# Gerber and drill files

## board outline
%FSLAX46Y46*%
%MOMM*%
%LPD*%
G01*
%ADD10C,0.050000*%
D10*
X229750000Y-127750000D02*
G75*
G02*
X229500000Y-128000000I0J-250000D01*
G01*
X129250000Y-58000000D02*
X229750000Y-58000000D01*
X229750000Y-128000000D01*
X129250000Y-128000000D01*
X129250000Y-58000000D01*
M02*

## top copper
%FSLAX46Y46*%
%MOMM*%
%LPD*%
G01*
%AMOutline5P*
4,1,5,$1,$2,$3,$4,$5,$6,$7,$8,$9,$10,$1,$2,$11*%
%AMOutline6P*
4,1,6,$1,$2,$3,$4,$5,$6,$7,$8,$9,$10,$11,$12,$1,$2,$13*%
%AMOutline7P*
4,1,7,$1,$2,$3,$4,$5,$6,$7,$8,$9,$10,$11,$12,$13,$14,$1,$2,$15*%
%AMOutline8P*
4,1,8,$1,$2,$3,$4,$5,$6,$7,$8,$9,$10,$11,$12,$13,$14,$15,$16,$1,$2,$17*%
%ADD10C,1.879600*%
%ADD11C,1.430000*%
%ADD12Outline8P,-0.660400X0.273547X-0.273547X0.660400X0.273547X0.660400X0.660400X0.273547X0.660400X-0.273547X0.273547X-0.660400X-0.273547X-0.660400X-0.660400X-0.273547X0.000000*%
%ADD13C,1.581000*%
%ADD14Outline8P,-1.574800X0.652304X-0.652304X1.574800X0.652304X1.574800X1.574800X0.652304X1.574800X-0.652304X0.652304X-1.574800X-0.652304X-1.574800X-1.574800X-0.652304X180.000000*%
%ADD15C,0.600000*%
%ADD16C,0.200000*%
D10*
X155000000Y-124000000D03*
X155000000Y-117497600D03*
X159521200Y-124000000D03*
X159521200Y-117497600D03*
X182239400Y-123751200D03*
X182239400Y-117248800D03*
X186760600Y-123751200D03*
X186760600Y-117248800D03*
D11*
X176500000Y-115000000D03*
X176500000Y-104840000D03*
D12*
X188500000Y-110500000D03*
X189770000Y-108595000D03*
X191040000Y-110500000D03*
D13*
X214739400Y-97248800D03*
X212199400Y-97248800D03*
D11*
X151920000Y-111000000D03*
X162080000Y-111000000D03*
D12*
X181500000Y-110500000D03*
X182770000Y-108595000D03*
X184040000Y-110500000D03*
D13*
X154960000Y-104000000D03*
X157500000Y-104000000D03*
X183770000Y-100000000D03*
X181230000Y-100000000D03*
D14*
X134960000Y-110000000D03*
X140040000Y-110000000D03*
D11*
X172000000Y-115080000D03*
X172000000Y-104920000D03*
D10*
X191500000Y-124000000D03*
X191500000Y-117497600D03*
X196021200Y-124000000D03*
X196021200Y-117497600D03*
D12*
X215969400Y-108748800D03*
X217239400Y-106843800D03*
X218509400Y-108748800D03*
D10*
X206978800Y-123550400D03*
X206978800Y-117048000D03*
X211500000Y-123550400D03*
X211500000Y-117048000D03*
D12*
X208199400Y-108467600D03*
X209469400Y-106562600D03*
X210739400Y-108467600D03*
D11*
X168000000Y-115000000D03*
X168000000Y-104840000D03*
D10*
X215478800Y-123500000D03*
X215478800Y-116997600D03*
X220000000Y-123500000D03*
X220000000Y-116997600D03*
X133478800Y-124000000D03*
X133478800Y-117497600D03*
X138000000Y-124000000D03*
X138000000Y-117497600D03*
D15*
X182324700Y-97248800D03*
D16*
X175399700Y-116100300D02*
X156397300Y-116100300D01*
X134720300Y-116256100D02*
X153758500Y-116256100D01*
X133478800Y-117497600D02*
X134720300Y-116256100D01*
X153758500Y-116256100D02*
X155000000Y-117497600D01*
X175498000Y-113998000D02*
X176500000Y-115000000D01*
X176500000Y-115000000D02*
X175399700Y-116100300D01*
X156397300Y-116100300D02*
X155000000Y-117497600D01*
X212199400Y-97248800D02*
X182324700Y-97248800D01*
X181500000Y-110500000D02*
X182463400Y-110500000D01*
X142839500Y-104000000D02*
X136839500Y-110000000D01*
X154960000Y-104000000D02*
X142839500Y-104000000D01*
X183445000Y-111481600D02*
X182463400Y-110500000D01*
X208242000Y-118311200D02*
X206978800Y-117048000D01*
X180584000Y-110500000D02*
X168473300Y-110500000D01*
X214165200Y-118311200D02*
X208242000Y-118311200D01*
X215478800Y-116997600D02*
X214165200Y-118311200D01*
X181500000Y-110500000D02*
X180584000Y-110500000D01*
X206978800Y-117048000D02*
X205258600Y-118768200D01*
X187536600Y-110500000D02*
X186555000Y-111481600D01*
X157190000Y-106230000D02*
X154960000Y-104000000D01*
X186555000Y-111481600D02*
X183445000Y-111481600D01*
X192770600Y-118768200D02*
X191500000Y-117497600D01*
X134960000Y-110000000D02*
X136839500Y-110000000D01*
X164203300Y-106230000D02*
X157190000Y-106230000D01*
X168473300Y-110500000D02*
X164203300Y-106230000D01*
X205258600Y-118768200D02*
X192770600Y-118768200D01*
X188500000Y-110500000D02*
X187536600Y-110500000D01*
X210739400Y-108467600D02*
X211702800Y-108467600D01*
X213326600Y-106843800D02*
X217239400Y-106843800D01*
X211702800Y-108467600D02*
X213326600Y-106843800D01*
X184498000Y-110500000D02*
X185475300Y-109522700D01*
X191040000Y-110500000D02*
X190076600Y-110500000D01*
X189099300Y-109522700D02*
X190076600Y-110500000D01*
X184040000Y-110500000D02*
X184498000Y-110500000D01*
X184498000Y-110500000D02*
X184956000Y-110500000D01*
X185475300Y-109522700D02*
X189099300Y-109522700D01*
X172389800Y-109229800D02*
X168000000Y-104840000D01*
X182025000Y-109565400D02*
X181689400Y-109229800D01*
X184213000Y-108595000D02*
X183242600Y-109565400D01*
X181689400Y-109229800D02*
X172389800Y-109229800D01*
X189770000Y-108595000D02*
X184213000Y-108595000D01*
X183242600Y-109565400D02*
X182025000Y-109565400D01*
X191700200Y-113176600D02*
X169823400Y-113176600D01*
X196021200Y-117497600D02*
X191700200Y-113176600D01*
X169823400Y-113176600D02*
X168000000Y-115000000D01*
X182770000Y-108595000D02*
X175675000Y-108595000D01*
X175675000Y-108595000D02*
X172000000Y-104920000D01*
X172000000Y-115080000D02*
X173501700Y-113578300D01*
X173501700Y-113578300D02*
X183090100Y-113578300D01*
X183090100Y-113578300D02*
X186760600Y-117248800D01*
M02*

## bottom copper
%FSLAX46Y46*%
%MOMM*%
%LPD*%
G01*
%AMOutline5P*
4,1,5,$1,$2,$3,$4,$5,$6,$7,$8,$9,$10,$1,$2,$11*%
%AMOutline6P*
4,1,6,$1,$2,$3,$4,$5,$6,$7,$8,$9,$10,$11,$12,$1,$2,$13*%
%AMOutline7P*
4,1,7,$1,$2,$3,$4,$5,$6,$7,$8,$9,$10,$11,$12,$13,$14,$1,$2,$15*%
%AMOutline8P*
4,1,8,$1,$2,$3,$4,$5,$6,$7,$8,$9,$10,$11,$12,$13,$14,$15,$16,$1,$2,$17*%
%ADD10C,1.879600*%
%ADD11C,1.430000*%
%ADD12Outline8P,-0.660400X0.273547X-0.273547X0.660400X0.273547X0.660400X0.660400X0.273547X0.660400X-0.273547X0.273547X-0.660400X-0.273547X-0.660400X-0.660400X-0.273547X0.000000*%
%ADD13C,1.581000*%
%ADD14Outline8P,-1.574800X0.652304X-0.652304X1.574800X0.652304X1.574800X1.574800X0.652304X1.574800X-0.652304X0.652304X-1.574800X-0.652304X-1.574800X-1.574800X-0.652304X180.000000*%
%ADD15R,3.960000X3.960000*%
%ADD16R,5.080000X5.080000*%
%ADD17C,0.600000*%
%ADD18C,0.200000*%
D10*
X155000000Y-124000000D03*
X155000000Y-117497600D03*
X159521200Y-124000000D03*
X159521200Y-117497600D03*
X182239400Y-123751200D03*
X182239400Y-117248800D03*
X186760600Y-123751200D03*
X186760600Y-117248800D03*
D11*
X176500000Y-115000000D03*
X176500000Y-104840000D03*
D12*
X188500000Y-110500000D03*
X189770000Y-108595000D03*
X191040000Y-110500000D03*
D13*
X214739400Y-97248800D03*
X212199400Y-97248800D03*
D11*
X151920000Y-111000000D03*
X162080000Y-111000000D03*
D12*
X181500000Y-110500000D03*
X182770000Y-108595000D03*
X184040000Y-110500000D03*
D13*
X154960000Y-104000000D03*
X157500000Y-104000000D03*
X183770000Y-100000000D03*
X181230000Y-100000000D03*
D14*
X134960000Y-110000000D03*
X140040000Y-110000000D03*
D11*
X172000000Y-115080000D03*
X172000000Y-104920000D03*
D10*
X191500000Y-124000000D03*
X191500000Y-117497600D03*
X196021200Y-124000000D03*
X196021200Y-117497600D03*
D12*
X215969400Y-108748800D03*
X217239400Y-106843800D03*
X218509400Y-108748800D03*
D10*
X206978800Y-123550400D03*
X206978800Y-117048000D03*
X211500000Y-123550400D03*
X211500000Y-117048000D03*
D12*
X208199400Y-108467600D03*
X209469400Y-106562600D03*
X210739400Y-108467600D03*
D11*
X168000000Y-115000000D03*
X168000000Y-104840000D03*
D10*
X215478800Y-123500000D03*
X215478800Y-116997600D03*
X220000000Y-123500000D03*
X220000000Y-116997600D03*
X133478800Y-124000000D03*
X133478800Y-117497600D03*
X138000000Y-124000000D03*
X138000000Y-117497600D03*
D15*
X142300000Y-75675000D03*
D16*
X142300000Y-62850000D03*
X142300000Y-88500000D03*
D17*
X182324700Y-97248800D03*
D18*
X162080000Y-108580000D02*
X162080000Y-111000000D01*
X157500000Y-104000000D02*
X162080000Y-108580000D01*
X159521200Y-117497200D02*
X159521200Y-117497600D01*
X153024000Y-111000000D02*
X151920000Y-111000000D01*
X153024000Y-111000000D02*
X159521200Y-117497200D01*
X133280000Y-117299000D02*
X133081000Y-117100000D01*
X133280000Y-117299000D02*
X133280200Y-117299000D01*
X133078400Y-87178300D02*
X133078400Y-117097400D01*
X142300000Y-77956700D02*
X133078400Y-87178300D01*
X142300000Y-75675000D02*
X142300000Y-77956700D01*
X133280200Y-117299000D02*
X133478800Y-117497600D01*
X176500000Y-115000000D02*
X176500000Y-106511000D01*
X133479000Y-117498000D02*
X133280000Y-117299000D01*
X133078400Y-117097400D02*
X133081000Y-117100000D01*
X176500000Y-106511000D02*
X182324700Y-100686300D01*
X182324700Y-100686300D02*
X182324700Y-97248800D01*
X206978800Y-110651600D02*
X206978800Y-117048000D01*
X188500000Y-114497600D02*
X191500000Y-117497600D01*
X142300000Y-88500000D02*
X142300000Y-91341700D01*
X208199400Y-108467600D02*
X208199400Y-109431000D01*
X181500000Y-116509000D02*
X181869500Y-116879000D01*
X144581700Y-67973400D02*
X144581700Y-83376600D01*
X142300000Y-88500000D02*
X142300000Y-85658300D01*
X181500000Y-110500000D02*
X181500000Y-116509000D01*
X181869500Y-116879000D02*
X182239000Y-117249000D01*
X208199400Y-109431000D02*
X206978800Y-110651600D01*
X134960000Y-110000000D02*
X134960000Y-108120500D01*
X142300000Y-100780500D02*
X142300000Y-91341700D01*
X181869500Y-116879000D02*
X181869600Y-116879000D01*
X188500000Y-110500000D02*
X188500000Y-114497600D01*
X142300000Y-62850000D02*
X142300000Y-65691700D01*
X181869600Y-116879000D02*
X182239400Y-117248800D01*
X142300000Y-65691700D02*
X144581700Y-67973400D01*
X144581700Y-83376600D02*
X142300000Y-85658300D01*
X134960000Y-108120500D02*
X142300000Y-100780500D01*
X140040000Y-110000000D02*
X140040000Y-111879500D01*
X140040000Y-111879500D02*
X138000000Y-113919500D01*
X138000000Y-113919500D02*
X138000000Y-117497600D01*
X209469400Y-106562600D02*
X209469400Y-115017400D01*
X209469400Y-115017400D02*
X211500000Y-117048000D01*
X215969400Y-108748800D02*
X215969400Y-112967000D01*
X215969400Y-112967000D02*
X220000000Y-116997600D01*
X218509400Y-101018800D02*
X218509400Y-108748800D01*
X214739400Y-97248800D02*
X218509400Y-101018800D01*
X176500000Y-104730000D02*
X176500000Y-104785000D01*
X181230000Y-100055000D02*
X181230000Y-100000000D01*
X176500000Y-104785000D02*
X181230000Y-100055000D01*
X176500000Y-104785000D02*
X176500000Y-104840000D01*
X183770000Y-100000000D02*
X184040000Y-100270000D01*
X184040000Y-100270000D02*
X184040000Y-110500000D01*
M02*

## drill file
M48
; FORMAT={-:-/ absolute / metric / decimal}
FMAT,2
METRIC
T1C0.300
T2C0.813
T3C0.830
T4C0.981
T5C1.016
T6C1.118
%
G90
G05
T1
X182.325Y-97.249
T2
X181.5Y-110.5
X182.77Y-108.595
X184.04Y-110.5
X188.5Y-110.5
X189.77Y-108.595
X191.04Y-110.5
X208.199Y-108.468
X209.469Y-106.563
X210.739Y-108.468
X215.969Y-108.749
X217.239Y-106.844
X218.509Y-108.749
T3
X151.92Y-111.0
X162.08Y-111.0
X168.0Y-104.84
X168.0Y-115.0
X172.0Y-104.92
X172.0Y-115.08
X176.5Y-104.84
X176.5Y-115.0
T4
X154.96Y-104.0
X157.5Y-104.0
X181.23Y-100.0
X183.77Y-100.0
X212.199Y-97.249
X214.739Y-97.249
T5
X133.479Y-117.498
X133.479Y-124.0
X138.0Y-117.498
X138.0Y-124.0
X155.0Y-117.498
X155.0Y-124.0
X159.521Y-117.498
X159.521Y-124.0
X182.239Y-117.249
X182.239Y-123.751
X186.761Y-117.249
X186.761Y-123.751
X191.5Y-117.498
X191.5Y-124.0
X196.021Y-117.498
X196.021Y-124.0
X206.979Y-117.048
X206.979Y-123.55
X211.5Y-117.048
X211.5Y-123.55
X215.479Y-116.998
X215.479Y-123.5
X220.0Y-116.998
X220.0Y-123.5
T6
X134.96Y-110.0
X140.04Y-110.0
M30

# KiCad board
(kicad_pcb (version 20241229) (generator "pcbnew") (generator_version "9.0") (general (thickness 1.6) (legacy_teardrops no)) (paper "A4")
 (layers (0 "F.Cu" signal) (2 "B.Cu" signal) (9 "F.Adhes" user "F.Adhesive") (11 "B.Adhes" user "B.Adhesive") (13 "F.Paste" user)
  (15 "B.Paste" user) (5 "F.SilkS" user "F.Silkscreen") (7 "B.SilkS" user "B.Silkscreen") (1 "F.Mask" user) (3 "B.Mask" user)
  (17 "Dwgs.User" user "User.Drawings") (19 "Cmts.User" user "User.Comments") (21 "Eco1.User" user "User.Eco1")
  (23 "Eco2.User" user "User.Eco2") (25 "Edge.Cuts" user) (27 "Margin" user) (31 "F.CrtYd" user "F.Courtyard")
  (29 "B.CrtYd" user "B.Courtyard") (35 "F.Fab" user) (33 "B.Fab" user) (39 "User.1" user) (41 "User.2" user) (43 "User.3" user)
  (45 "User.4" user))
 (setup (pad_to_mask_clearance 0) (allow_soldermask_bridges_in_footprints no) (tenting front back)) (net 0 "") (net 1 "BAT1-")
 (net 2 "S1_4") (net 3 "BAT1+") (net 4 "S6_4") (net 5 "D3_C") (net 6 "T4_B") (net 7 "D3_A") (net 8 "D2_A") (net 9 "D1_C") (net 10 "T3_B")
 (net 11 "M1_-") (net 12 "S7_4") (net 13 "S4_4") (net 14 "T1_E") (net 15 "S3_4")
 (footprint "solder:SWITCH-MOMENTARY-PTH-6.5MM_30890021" (layer "F.Cu") (at 157.2606 120.7488 90)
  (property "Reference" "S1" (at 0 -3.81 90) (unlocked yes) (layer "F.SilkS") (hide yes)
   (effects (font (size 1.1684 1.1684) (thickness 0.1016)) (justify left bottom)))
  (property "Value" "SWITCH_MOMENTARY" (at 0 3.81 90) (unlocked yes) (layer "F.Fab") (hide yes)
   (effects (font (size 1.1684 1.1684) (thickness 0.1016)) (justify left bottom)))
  (pad "1" thru_hole circle (at -3.2512 -2.2606 90) (size 1.8796 1.8796) (drill 1.016) (layers "*.Cu" "*.Mask") (remove_unused_layers no)
   (solder_mask_margin 0.1016) (thermal_bridge_angle 0))
  (pad "2" thru_hole circle (at 3.2512 -2.2606 90) (size 1.8796 1.8796) (drill 1.016) (layers "*.Cu" "*.Mask") (remove_unused_layers no)
   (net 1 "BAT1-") (solder_mask_margin 0.1016) (thermal_bridge_angle 0))
  (pad "3" thru_hole circle (at -3.2512 2.2606 90) (size 1.8796 1.8796) (drill 1.016) (layers "*.Cu" "*.Mask") (remove_unused_layers no)
   (solder_mask_margin 0.1016) (thermal_bridge_angle 0))
  (pad "4" thru_hole circle (at 3.2512 2.2606 90) (size 1.8796 1.8796) (drill 1.016) (layers "*.Cu" "*.Mask") (remove_unused_layers no)
   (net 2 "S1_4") (solder_mask_margin 0.1016) (thermal_bridge_angle 0)))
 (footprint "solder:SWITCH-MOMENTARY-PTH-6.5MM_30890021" (layer "F.Cu") (at 184.5 120.5 90)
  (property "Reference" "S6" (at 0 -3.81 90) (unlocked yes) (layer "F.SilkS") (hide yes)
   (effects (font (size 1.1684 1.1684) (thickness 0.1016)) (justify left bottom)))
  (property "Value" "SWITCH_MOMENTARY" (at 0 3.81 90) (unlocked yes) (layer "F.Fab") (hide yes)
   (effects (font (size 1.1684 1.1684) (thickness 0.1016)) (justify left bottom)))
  (pad "1" thru_hole circle (at -3.2512 -2.2606 90) (size 1.8796 1.8796) (drill 1.016) (layers "*.Cu" "*.Mask") (remove_unused_layers no)
   (solder_mask_margin 0.1016) (thermal_bridge_angle 0))
  (pad "2" thru_hole circle (at 3.2512 -2.2606 90) (size 1.8796 1.8796) (drill 1.016) (layers "*.Cu" "*.Mask") (remove_unused_layers no)
   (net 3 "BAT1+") (solder_mask_margin 0.1016) (thermal_bridge_angle 0))
  (pad "3" thru_hole circle (at -3.2512 2.2606 90) (size 1.8796 1.8796) (drill 1.016) (layers "*.Cu" "*.Mask") (remove_unused_layers no)
   (solder_mask_margin 0.1016) (thermal_bridge_angle 0))
  (pad "4" thru_hole circle (at 3.2512 2.2606 90) (size 1.8796 1.8796) (drill 1.016) (layers "*.Cu" "*.Mask") (remove_unused_layers no)
   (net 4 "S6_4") (solder_mask_margin 0.1016) (thermal_bridge_angle 0)))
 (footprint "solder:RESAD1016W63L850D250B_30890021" (layer "F.Cu") (at 176.5 109.92 90)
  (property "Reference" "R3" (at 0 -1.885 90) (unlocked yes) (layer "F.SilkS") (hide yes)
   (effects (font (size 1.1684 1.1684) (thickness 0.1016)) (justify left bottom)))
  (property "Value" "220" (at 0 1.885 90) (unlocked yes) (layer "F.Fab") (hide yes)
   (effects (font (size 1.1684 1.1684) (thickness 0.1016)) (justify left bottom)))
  (pad "1" thru_hole circle (at -5.08 0 90) (size 1.43 1.43) (drill 0.83) (layers "*.Cu" "*.Mask") (remove_unused_layers no) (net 1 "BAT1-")
   (solder_mask_margin 0.1016) (thermal_bridge_angle 0))
  (pad "2" thru_hole circle (at 5.08 0 90) (size 1.43 1.43) (drill 0.83) (layers "*.Cu" "*.Mask") (remove_unused_layers no) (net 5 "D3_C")
   (solder_mask_margin 0.1016) (thermal_bridge_angle 0)))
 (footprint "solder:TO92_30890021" (layer "F.Cu") (at 189.77 110.5)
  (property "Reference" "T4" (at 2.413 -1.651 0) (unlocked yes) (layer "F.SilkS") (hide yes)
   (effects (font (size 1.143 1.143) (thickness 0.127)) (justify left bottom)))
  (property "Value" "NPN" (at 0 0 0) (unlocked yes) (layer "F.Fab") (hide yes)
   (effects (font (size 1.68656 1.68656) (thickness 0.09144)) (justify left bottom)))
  (pad "1" thru_hole roundrect (at -1.27 0) (size 1.3208 1.3208) (drill 0.8128) (layers "*.Cu" "*.Mask") (remove_unused_layers no)
   (roundrect_rratio 0.25) (chamfer_ratio 0.2928932188) (chamfer top_left top_right bottom_left bottom_right) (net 3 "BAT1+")
   (solder_mask_margin 0.1016) (thermal_bridge_angle 0))
  (pad "2" thru_hole roundrect (at 0 -1.905) (size 1.3208 1.3208) (drill 0.8128) (layers "*.Cu" "*.Mask") (remove_unused_layers no)
   (roundrect_rratio 0.25) (chamfer_ratio 0.2928932188) (chamfer top_left top_right bottom_left bottom_right) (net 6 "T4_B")
   (solder_mask_margin 0.1016) (thermal_bridge_angle 0))
  (pad "3" thru_hole roundrect (at 1.27 0) (size 1.3208 1.3208) (drill 0.8128) (layers "*.Cu" "*.Mask") (remove_unused_layers no)
   (roundrect_rratio 0.25) (chamfer_ratio 0.2928932188) (chamfer top_left top_right bottom_left bottom_right) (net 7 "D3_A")
   (solder_mask_margin 0.1016) (thermal_bridge_angle 0)))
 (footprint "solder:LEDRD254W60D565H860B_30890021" (layer "F.Cu") (at 213.4694 97.2488 180)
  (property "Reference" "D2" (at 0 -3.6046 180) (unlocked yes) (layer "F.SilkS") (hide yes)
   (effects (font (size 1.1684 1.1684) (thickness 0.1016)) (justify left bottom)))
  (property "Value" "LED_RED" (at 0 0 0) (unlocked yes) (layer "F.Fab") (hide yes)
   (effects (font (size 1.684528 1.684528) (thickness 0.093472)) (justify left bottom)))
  (pad "1" thru_hole circle (at -1.27 0 180) (size 1.581 1.581) (drill 0.981) (layers "*.Cu" "*.Mask") (remove_unused_layers no)
   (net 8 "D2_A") (solder_mask_margin 0.1016) (thermal_bridge_angle 0))
  (pad "2" thru_hole circle (at 1.27 0 180) (size 1.581 1.581) (drill 0.981) (layers "*.Cu" "*.Mask") (remove_unused_layers no)
   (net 1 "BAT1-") (solder_mask_margin 0.1016) (thermal_bridge_angle 0)))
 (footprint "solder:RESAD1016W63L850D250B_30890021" (layer "F.Cu") (at 157 111)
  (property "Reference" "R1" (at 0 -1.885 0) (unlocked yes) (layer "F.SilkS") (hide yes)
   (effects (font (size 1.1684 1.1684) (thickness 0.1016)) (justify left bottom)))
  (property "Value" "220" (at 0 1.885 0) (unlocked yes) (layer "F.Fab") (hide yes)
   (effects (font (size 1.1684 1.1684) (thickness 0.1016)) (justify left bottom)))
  (pad "1" thru_hole circle (at -5.08 0) (size 1.43 1.43) (drill 0.83) (layers "*.Cu" "*.Mask") (remove_unused_layers no) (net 2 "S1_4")
   (solder_mask_margin 0.1016) (thermal_bridge_angle 0))
  (pad "2" thru_hole circle (at 5.08 0) (size 1.43 1.43) (drill 0.83) (layers "*.Cu" "*.Mask") (remove_unused_layers no) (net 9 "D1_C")
   (solder_mask_margin 0.1016) (thermal_bridge_angle 0)))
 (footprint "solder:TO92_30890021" (layer "F.Cu") (at 182.77 110.5)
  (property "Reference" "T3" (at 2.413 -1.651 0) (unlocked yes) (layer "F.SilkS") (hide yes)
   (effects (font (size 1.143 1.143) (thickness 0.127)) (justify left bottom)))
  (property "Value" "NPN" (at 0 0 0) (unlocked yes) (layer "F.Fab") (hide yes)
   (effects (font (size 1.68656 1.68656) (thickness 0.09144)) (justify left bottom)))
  (pad "1" thru_hole roundrect (at -1.27 0) (size 1.3208 1.3208) (drill 0.8128) (layers "*.Cu" "*.Mask") (remove_unused_layers no)
   (roundrect_rratio 0.25) (chamfer_ratio 0.2928932188) (chamfer top_left top_right bottom_left bottom_right) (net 3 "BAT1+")
   (solder_mask_margin 0.1016) (thermal_bridge_angle 0))
  (pad "2" thru_hole roundrect (at 0 -1.905) (size 1.3208 1.3208) (drill 0.8128) (layers "*.Cu" "*.Mask") (remove_unused_layers no)
   (roundrect_rratio 0.25) (chamfer_ratio 0.2928932188) (chamfer top_left top_right bottom_left bottom_right) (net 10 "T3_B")
   (solder_mask_margin 0.1016) (thermal_bridge_angle 0))
  (pad "3" thru_hole roundrect (at 1.27 0) (size 1.3208 1.3208) (drill 0.8128) (layers "*.Cu" "*.Mask") (remove_unused_layers no)
   (roundrect_rratio 0.25) (chamfer_ratio 0.2928932188) (chamfer top_left top_right bottom_left bottom_right) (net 7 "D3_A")
   (solder_mask_margin 0.1016) (thermal_bridge_angle 0)))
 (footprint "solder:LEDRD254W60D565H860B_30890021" (layer "F.Cu") (at 156.23 104)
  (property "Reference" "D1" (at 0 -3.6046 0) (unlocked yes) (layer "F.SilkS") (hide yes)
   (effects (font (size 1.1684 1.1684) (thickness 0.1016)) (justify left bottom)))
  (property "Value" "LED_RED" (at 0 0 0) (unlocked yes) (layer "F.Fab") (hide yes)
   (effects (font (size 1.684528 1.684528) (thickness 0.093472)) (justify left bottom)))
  (pad "1" thru_hole circle (at -1.27 0) (size 1.581 1.581) (drill 0.981) (layers "*.Cu" "*.Mask") (remove_unused_layers no) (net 3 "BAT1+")
   (solder_mask_margin 0.1016) (thermal_bridge_angle 0))
  (pad "2" thru_hole circle (at 1.27 0) (size 1.581 1.581) (drill 0.981) (layers "*.Cu" "*.Mask") (remove_unused_layers no) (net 9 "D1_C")
   (solder_mask_margin 0.1016) (thermal_bridge_angle 0)))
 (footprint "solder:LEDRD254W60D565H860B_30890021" (layer "F.Cu") (at 182.5 100 180)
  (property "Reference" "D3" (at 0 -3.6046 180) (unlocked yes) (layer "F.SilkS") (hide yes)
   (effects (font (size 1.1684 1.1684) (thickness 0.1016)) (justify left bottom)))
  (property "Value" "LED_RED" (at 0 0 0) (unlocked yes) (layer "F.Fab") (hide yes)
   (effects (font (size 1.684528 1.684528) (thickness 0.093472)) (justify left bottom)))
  (pad "1" thru_hole circle (at -1.27 0 180) (size 1.581 1.581) (drill 0.981) (layers "*.Cu" "*.Mask") (remove_unused_layers no)
   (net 7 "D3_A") (solder_mask_margin 0.1016) (thermal_bridge_angle 0))
  (pad "2" thru_hole circle (at 1.27 0 180) (size 1.581 1.581) (drill 0.981) (layers "*.Cu" "*.Mask") (remove_unused_layers no)
   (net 5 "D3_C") (solder_mask_margin 0.1016) (thermal_bridge_angle 0)))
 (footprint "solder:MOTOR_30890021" (layer "F.Cu") (at 137.5 110 180)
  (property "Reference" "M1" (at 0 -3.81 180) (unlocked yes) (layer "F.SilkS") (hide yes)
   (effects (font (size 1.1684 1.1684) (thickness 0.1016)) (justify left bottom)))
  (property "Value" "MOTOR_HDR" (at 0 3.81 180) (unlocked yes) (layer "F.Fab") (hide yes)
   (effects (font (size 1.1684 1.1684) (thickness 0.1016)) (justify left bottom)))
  (pad "+" thru_hole roundrect (at 2.54 0 180) (size 3.1496 3.1496) (drill 1.1176) (layers "*.Cu" "*.Mask") (remove_unused_layers no)
   (roundrect_rratio 0.25) (chamfer_ratio 0.2928932188) (chamfer top_left top_right bottom_left bottom_right) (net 3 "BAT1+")
   (solder_mask_margin 0.1016) (thermal_bridge_angle 0))
  (pad "-" thru_hole roundrect (at -2.54 0 180) (size 3.1496 3.1496) (drill 1.1176) (layers "*.Cu" "*.Mask") (remove_unused_layers no)
   (roundrect_rratio 0.25) (chamfer_ratio 0.2928932188) (chamfer top_left top_right bottom_left bottom_right) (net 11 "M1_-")
   (solder_mask_margin 0.1016) (thermal_bridge_angle 0)))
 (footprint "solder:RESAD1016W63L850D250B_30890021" (layer "F.Cu") (at 172 110 90)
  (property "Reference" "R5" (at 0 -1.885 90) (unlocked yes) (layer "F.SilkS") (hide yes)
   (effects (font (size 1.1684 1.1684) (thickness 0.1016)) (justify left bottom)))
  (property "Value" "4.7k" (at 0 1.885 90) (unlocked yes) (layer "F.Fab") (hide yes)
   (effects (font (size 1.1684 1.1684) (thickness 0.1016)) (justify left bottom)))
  (pad "1" thru_hole circle (at -5.08 0 90) (size 1.43 1.43) (drill 0.83) (layers "*.Cu" "*.Mask") (remove_unused_layers no) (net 4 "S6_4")
   (solder_mask_margin 0.1016) (thermal_bridge_angle 0))
  (pad "2" thru_hole circle (at 5.08 0 90) (size 1.43 1.43) (drill 0.83) (layers "*.Cu" "*.Mask") (remove_unused_layers no) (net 10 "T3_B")
   (solder_mask_margin 0.1016) (thermal_bridge_angle 0)))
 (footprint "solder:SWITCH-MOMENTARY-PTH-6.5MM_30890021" (layer "F.Cu") (at 193.7606 120.7488 90)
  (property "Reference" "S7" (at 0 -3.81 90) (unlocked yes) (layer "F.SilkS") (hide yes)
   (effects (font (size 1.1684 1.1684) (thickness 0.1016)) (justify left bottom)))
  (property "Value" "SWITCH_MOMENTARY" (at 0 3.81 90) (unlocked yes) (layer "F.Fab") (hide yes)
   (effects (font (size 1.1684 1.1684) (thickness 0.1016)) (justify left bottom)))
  (pad "1" thru_hole circle (at -3.2512 -2.2606 90) (size 1.8796 1.8796) (drill 1.016) (layers "*.Cu" "*.Mask") (remove_unused_layers no)
   (solder_mask_margin 0.1016) (thermal_bridge_angle 0))
  (pad "2" thru_hole circle (at 3.2512 -2.2606 90) (size 1.8796 1.8796) (drill 1.016) (layers "*.Cu" "*.Mask") (remove_unused_layers no)
   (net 3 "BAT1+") (solder_mask_margin 0.1016) (thermal_bridge_angle 0))
  (pad "3" thru_hole circle (at -3.2512 2.2606 90) (size 1.8796 1.8796) (drill 1.016) (layers "*.Cu" "*.Mask") (remove_unused_layers no)
   (solder_mask_margin 0.1016) (thermal_bridge_angle 0))
  (pad "4" thru_hole circle (at 3.2512 2.2606 90) (size 1.8796 1.8796) (drill 1.016) (layers "*.Cu" "*.Mask") (remove_unused_layers no)
   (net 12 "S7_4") (solder_mask_margin 0.1016) (thermal_bridge_angle 0)))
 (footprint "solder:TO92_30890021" (layer "F.Cu") (at 217.2394 108.7488)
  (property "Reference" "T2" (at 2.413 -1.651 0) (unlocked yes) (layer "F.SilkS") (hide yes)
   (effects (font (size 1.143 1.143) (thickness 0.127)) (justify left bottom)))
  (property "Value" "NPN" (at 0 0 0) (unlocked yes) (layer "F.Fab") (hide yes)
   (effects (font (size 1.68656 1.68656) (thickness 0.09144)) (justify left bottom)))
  (pad "1" thru_hole roundrect (at -1.27 0) (size 1.3208 1.3208) (drill 0.8128) (layers "*.Cu" "*.Mask") (remove_unused_layers no)
   (roundrect_rratio 0.25) (chamfer_ratio 0.2928932188) (chamfer top_left top_right bottom_left bottom_right) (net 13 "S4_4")
   (solder_mask_margin 0.1016) (thermal_bridge_angle 0))
  (pad "2" thru_hole roundrect (at 0 -1.905) (size 1.3208 1.3208) (drill 0.8128) (layers "*.Cu" "*.Mask") (remove_unused_layers no)
   (roundrect_rratio 0.25) (chamfer_ratio 0.2928932188) (chamfer top_left top_right bottom_left bottom_right) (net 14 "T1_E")
   (solder_mask_margin 0.1016) (thermal_bridge_angle 0))
  (pad "3" thru_hole roundrect (at 1.27 0) (size 1.3208 1.3208) (drill 0.8128) (layers "*.Cu" "*.Mask") (remove_unused_layers no)
   (roundrect_rratio 0.25) (chamfer_ratio 0.2928932188) (chamfer top_left top_right bottom_left bottom_right) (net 8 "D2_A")
   (solder_mask_margin 0.1016) (thermal_bridge_angle 0)))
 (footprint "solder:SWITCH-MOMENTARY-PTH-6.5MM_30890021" (layer "F.Cu") (at 209.2394 120.2992 90)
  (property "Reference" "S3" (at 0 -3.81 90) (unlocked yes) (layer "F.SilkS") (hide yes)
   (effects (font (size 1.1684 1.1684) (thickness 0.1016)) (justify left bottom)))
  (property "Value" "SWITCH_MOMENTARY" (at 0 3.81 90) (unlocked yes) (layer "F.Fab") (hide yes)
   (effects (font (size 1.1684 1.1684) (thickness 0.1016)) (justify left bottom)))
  (pad "1" thru_hole circle (at -3.2512 -2.2606 90) (size 1.8796 1.8796) (drill 1.016) (layers "*.Cu" "*.Mask") (remove_unused_layers no)
   (solder_mask_margin 0.1016) (thermal_bridge_angle 0))
  (pad "2" thru_hole circle (at 3.2512 -2.2606 90) (size 1.8796 1.8796) (drill 1.016) (layers "*.Cu" "*.Mask") (remove_unused_layers no)
   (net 3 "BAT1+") (solder_mask_margin 0.1016) (thermal_bridge_angle 0))
  (pad "3" thru_hole circle (at -3.2512 2.2606 90) (size 1.8796 1.8796) (drill 1.016) (layers "*.Cu" "*.Mask") (remove_unused_layers no)
   (solder_mask_margin 0.1016) (thermal_bridge_angle 0))
  (pad "4" thru_hole circle (at 3.2512 2.2606 90) (size 1.8796 1.8796) (drill 1.016) (layers "*.Cu" "*.Mask") (remove_unused_layers no)
   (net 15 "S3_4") (solder_mask_margin 0.1016) (thermal_bridge_angle 0)))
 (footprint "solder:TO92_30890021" (layer "F.Cu") (at 209.4694 108.4676)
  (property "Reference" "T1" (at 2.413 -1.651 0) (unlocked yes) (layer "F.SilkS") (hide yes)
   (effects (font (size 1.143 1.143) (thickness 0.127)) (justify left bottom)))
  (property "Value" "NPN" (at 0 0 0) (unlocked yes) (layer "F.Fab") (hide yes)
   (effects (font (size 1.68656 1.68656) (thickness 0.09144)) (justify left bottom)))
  (pad "1" thru_hole roundrect (at -1.27 0) (size 1.3208 1.3208) (drill 0.8128) (layers "*.Cu" "*.Mask") (remove_unused_layers no)
   (roundrect_rratio 0.25) (chamfer_ratio 0.2928932188) (chamfer top_left top_right bottom_left bottom_right) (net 3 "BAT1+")
   (solder_mask_margin 0.1016) (thermal_bridge_angle 0))
  (pad "2" thru_hole roundrect (at 0 -1.905) (size 1.3208 1.3208) (drill 0.8128) (layers "*.Cu" "*.Mask") (remove_unused_layers no)
   (roundrect_rratio 0.25) (chamfer_ratio 0.2928932188) (chamfer top_left top_right bottom_left bottom_right) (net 15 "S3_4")
   (solder_mask_margin 0.1016) (thermal_bridge_angle 0))
  (pad "3" thru_hole roundrect (at 1.27 0) (size 1.3208 1.3208) (drill 0.8128) (layers "*.Cu" "*.Mask") (remove_unused_layers no)
   (roundrect_rratio 0.25) (chamfer_ratio 0.2928932188) (chamfer top_left top_right bottom_left bottom_right) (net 14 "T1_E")
   (solder_mask_margin 0.1016) (thermal_bridge_angle 0)))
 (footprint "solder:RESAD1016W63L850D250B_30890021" (layer "F.Cu") (at 168 109.92 90)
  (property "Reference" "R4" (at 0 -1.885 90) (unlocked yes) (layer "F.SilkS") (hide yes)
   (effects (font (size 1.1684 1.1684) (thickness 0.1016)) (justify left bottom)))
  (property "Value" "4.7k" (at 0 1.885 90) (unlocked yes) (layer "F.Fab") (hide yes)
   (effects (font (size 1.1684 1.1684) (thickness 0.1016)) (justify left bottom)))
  (pad "1" thru_hole circle (at -5.08 0 90) (size 1.43 1.43) (drill 0.83) (layers "*.Cu" "*.Mask") (remove_unused_layers no) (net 12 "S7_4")
   (solder_mask_margin 0.1016) (thermal_bridge_angle 0))
  (pad "2" thru_hole circle (at 5.08 0 90) (size 1.43 1.43) (drill 0.83) (layers "*.Cu" "*.Mask") (remove_unused_layers no) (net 6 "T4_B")
   (solder_mask_margin 0.1016) (thermal_bridge_angle 0)))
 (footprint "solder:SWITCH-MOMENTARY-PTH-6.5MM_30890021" (layer "F.Cu") (at 217.7394 120.2488 90)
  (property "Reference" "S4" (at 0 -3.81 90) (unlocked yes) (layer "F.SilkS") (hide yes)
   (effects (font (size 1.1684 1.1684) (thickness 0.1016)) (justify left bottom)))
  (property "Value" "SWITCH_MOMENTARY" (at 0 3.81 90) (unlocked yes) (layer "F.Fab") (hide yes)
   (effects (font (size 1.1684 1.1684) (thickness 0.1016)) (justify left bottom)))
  (pad "1" thru_hole circle (at -3.2512 -2.2606 90) (size 1.8796 1.8796) (drill 1.016) (layers "*.Cu" "*.Mask") (remove_unused_layers no)
   (solder_mask_margin 0.1016) (thermal_bridge_angle 0))
  (pad "2" thru_hole circle (at 3.2512 -2.2606 90) (size 1.8796 1.8796) (drill 1.016) (layers "*.Cu" "*.Mask") (remove_unused_layers no)
   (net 3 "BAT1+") (solder_mask_margin 0.1016) (thermal_bridge_angle 0))
  (pad "3" thru_hole circle (at -3.2512 2.2606 90) (size 1.8796 1.8796) (drill 1.016) (layers "*.Cu" "*.Mask") (remove_unused_layers no)
   (solder_mask_margin 0.1016) (thermal_bridge_angle 0))
  (pad "4" thru_hole circle (at 3.2512 2.2606 90) (size 1.8796 1.8796) (drill 1.016) (layers "*.Cu" "*.Mask") (remove_unused_layers no)
   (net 13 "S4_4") (solder_mask_margin 0.1016) (thermal_bridge_angle 0)))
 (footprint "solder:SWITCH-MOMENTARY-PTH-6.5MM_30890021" (layer "F.Cu") (at 135.7394 120.7488 90)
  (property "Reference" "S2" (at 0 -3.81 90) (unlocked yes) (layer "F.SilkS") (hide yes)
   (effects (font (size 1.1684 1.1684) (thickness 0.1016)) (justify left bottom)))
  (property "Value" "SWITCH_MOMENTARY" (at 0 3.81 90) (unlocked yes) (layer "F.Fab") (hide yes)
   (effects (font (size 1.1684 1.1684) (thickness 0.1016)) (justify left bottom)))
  (pad "1" thru_hole circle (at -3.2512 -2.2606 90) (size 1.8796 1.8796) (drill 1.016) (layers "*.Cu" "*.Mask") (remove_unused_layers no)
   (solder_mask_margin 0.1016) (thermal_bridge_angle 0))
  (pad "2" thru_hole circle (at 3.2512 -2.2606 90) (size 1.8796 1.8796) (drill 1.016) (layers "*.Cu" "*.Mask") (remove_unused_layers no)
   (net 1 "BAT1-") (solder_mask_margin 0.1016) (thermal_bridge_angle 0))
  (pad "3" thru_hole circle (at -3.2512 2.2606 90) (size 1.8796 1.8796) (drill 1.016) (layers "*.Cu" "*.Mask") (remove_unused_layers no)
   (solder_mask_margin 0.1016) (thermal_bridge_angle 0))
  (pad "4" thru_hole circle (at 3.2512 2.2606 90) (size 1.8796 1.8796) (drill 1.016) (layers "*.Cu" "*.Mask") (remove_unused_layers no)
   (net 11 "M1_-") (solder_mask_margin 0.1016) (thermal_bridge_angle 0)))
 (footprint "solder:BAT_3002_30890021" (layer "B.Cu") (at 141.65 75.675 90)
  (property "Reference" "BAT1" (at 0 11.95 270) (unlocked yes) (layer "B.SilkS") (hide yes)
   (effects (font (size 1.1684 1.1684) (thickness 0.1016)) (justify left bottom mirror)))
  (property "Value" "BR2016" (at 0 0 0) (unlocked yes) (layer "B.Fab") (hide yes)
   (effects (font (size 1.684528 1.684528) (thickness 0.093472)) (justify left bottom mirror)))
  (pad "N" smd rect (at 0 0.65 90) (size 3.96 3.96) (layers "B.Cu" "B.Mask" "B.Paste") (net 1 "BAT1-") (solder_mask_margin 0.1016)
   (solder_paste_margin 0) (thermal_bridge_angle 0))
  (pad "P" smd rect (at 12.825 0.65 90) (size 5.08 5.08) (layers "B.Cu" "B.Mask" "B.Paste") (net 3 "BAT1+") (solder_mask_margin 0.1016)
   (solder_paste_margin 0) (thermal_bridge_angle 0))
  (pad "P1" smd rect (at -12.825 0.65 90) (size 5.08 5.08) (layers "B.Cu" "B.Mask" "B.Paste") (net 3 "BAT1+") (solder_mask_margin 0.1016)
   (solder_paste_margin 0) (thermal_bridge_angle 0)))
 (gr_arc (start 229.75 127.75) (mid 229.926777 128.176777) (end 229.5 128) (stroke (width 0.05) (type default)) (layer "Edge.Cuts"))
 (gr_rect (start 129.25 58) (end 229.75 128) (stroke (width 0.05) (type default)) (fill no) (layer "Edge.Cuts"))
 (segment (start 162.08 108.58) (end 162.08 111) (width 0.2) (layer "B.Cu") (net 9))
 (segment (start 157.5 104) (end 162.08 108.58) (width 0.2) (layer "B.Cu") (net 9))
 (segment (start 159.5212 117.4972) (end 159.5212 117.4976) (width 0.2) (layer "B.Cu") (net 2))
 (segment (start 153.024 111) (end 151.92 111) (width 0.2) (layer "B.Cu") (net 2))
 (segment (start 153.024 111) (end 159.5212 117.4972) (width 0.2) (layer "B.Cu") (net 2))
 (segment (start 175.3997 116.1003) (end 156.3973 116.1003) (width 0.2) (layer "F.Cu") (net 1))
 (segment (start 134.7203 116.2561) (end 153.7585 116.2561) (width 0.2) (layer "F.Cu") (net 1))
 (segment (start 133.4788 117.4976) (end 134.7203 116.2561) (width 0.2) (layer "F.Cu") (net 1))
 (segment (start 153.7585 116.2561) (end 155 117.4976) (width 0.2) (layer "F.Cu") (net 1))
 (segment (start 175.498 113.998) (end 176.5 115) (width 0.2) (layer "F.Cu") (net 1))
 (segment (start 176.5 115) (end 175.3997 116.1003) (width 0.2) (layer "F.Cu") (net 1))
 (segment (start 156.3973 116.1003) (end 155 117.4976) (width 0.2) (layer "F.Cu") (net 1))
 (segment (start 212.1994 97.2488) (end 182.3247 97.2488) (width 0.2) (layer "F.Cu") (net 1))
 (via (at 182.3247 97.2488) (size 0.6) (drill 0.3) (layers "F.Cu" "B.Cu") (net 1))
 (segment (start 133.28 117.299) (end 133.081 117.1) (width 0.2) (layer "B.Cu") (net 1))
 (segment (start 133.28 117.299) (end 133.2802 117.299) (width 0.2) (layer "B.Cu") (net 1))
 (segment (start 133.0784 87.1783) (end 133.0784 117.0974) (width 0.2) (layer "B.Cu") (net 1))
 (segment (start 142.3 77.9567) (end 133.0784 87.1783) (width 0.2) (layer "B.Cu") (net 1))
 (segment (start 142.3 75.675) (end 142.3 77.9567) (width 0.2) (layer "B.Cu") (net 1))
 (segment (start 133.2802 117.299) (end 133.4788 117.4976) (width 0.2) (layer "B.Cu") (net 1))
 (segment (start 176.5 115) (end 176.5 106.511) (width 0.2) (layer "B.Cu") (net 1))
 (segment (start 133.479 117.498) (end 133.28 117.299) (width 0.2) (layer "B.Cu") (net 1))
 (segment (start 133.0784 117.0974) (end 133.081 117.1) (width 0.2) (layer "B.Cu") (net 1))
 (segment (start 176.5 106.511) (end 182.3247 100.6863) (width 0.2) (layer "B.Cu") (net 1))
 (segment (start 182.3247 100.6863) (end 182.3247 97.2488) (width 0.2) (layer "B.Cu") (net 1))
 (segment (start 181.5 110.5) (end 182.4634 110.5) (width 0.2) (layer "F.Cu") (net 3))
 (segment (start 142.8395 104) (end 136.8395 110) (width 0.2) (layer "F.Cu") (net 3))
 (segment (start 154.96 104) (end 142.8395 104) (width 0.2) (layer "F.Cu") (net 3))
 (segment (start 183.445 111.4816) (end 182.4634 110.5) (width 0.2) (layer "F.Cu") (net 3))
 (segment (start 208.242 118.3112) (end 206.9788 117.048) (width 0.2) (layer "F.Cu") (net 3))
 (segment (start 180.584 110.5) (end 168.4733 110.5) (width 0.2) (layer "F.Cu") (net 3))
 (segment (start 214.1652 118.3112) (end 208.242 118.3112) (width 0.2) (layer "F.Cu") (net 3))
 (segment (start 215.4788 116.9976) (end 214.1652 118.3112) (width 0.2) (layer "F.Cu") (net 3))
 (segment (start 181.5 110.5) (end 180.584 110.5) (width 0.2) (layer "F.Cu") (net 3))
 (segment (start 206.9788 117.048) (end 205.2586 118.7682) (width 0.2) (layer "F.Cu") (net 3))
 (segment (start 187.5366 110.5) (end 186.555 111.4816) (width 0.2) (layer "F.Cu") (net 3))
 (segment (start 157.19 106.23) (end 154.96 104) (width 0.2) (layer "F.Cu") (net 3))
 (segment (start 186.555 111.4816) (end 183.445 111.4816) (width 0.2) (layer "F.Cu") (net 3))
 (segment (start 192.7706 118.7682) (end 191.5 117.4976) (width 0.2) (layer "F.Cu") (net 3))
 (segment (start 134.96 110) (end 136.8395 110) (width 0.2) (layer "F.Cu") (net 3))
 (segment (start 164.2033 106.23) (end 157.19 106.23) (width 0.2) (layer "F.Cu") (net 3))
 (segment (start 168.4733 110.5) (end 164.2033 106.23) (width 0.2) (layer "F.Cu") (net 3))
 (segment (start 205.2586 118.7682) (end 192.7706 118.7682) (width 0.2) (layer "F.Cu") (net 3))
 (segment (start 188.5 110.5) (end 187.5366 110.5) (width 0.2) (layer "F.Cu") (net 3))
 (segment (start 206.9788 110.6516) (end 206.9788 117.048) (width 0.2) (layer "B.Cu") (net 3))
 (segment (start 188.5 114.4976) (end 191.5 117.4976) (width 0.2) (layer "B.Cu") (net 3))
 (segment (start 142.3 88.5) (end 142.3 91.3417) (width 0.2) (layer "B.Cu") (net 3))
 (segment (start 208.1994 108.4676) (end 208.1994 109.431) (width 0.2) (layer "B.Cu") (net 3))
 (segment (start 181.5 116.509) (end 181.8695 116.879) (width 0.2) (layer "B.Cu") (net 3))
 (segment (start 144.5817 67.9734) (end 144.5817 83.3766) (width 0.2) (layer "B.Cu") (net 3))
 (segment (start 142.3 88.5) (end 142.3 85.6583) (width 0.2) (layer "B.Cu") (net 3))
 (segment (start 181.5 110.5) (end 181.5 116.509) (width 0.2) (layer "B.Cu") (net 3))
 (segment (start 181.8695 116.879) (end 182.239 117.249) (width 0.2) (layer "B.Cu") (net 3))
 (segment (start 208.1994 109.431) (end 206.9788 110.6516) (width 0.2) (layer "B.Cu") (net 3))
 (segment (start 134.96 110) (end 134.96 108.1205) (width 0.2) (layer "B.Cu") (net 3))
 (segment (start 142.3 100.7805) (end 142.3 91.3417) (width 0.2) (layer "B.Cu") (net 3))
 (segment (start 181.8695 116.879) (end 181.8696 116.879) (width 0.2) (layer "B.Cu") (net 3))
 (segment (start 188.5 110.5) (end 188.5 114.4976) (width 0.2) (layer "B.Cu") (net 3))
 (segment (start 142.3 62.85) (end 142.3 65.6917) (width 0.2) (layer "B.Cu") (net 3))
 (segment (start 181.8696 116.879) (end 182.2394 117.2488) (width 0.2) (layer "B.Cu") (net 3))
 (segment (start 142.3 65.6917) (end 144.5817 67.9734) (width 0.2) (layer "B.Cu") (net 3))
 (segment (start 144.5817 83.3766) (end 142.3 85.6583) (width 0.2) (layer "B.Cu") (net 3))
 (segment (start 134.96 108.1205) (end 142.3 100.7805) (width 0.2) (layer "B.Cu") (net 3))
 (segment (start 140.04 110) (end 140.04 111.8795) (width 0.2) (layer "B.Cu") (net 11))
 (segment (start 140.04 111.8795) (end 138 113.9195) (width 0.2) (layer "B.Cu") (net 11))
 (segment (start 138 113.9195) (end 138 117.4976) (width 0.2) (layer "B.Cu") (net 11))
 (segment (start 209.4694 106.5626) (end 209.4694 115.0174) (width 0.2) (layer "B.Cu") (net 15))
 (segment (start 209.4694 115.0174) (end 211.5 117.048) (width 0.2) (layer "B.Cu") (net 15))
 (segment (start 210.7394 108.4676) (end 211.7028 108.4676) (width 0.2) (layer "F.Cu") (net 14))
 (segment (start 213.3266 106.8438) (end 217.2394 106.8438) (width 0.2) (layer "F.Cu") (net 14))
 (segment (start 211.7028 108.4676) (end 213.3266 106.8438) (width 0.2) (layer "F.Cu") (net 14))
 (segment (start 215.9694 108.7488) (end 215.9694 112.967) (width 0.2) (layer "B.Cu") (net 13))
 (segment (start 215.9694 112.967) (end 220 116.9976) (width 0.2) (layer "B.Cu") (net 13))
 (segment (start 218.5094 101.0188) (end 218.5094 108.7488) (width 0.2) (layer "B.Cu") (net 8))
 (segment (start 214.7394 97.2488) (end 218.5094 101.0188) (width 0.2) (layer "B.Cu") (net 8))
 (segment (start 176.5 104.73) (end 176.5 104.785) (width 0.2) (layer "B.Cu") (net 5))
 (segment (start 181.23 100.055) (end 181.23 100) (width 0.2) (layer "B.Cu") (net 5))
 (segment (start 176.5 104.785) (end 181.23 100.055) (width 0.2) (layer "B.Cu") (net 5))
 (segment (start 176.5 104.785) (end 176.5 104.84) (width 0.2) (layer "B.Cu") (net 5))
 (segment (start 184.498 110.5) (end 185.4753 109.5227) (width 0.2) (layer "F.Cu") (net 7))
 (segment (start 191.04 110.5) (end 190.0766 110.5) (width 0.2) (layer "F.Cu") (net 7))
 (segment (start 189.0993 109.5227) (end 190.0766 110.5) (width 0.2) (layer "F.Cu") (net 7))
 (segment (start 184.04 110.5) (end 184.498 110.5) (width 0.2) (layer "F.Cu") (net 7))
 (segment (start 184.498 110.5) (end 184.956 110.5) (width 0.2) (layer "F.Cu") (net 7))
 (segment (start 185.4753 109.5227) (end 189.0993 109.5227) (width 0.2) (layer "F.Cu") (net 7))
 (segment (start 183.77 100) (end 184.04 100.27) (width 0.2) (layer "B.Cu") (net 7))
 (segment (start 184.04 100.27) (end 184.04 110.5) (width 0.2) (layer "B.Cu") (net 7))
 (segment (start 172.3898 109.2298) (end 168 104.84) (width 0.2) (layer "F.Cu") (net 6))
 (segment (start 182.025 109.5654) (end 181.6894 109.2298) (width 0.2) (layer "F.Cu") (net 6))
 (segment (start 184.213 108.595) (end 183.2426 109.5654) (width 0.2) (layer "F.Cu") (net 6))
 (segment (start 181.6894 109.2298) (end 172.3898 109.2298) (width 0.2) (layer "F.Cu") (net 6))
 (segment (start 189.77 108.595) (end 184.213 108.595) (width 0.2) (layer "F.Cu") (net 6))
 (segment (start 183.2426 109.5654) (end 182.025 109.5654) (width 0.2) (layer "F.Cu") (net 6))
 (segment (start 191.7002 113.1766) (end 169.8234 113.1766) (width 0.2) (layer "F.Cu") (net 12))
 (segment (start 196.0212 117.4976) (end 191.7002 113.1766) (width 0.2) (layer "F.Cu") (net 12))
 (segment (start 169.8234 113.1766) (end 168 115) (width 0.2) (layer "F.Cu") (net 12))
 (segment (start 182.77 108.595) (end 175.675 108.595) (width 0.2) (layer "F.Cu") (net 10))
 (segment (start 175.675 108.595) (end 172 104.92) (width 0.2) (layer "F.Cu") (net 10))
 (segment (start 172 115.08) (end 173.5017 113.5783) (width 0.2) (layer "F.Cu") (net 4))
 (segment (start 173.5017 113.5783) (end 183.0901 113.5783) (width 0.2) (layer "F.Cu") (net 4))
 (segment (start 183.0901 113.5783) (end 186.7606 117.2488) (width 0.2) (layer "F.Cu") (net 4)))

